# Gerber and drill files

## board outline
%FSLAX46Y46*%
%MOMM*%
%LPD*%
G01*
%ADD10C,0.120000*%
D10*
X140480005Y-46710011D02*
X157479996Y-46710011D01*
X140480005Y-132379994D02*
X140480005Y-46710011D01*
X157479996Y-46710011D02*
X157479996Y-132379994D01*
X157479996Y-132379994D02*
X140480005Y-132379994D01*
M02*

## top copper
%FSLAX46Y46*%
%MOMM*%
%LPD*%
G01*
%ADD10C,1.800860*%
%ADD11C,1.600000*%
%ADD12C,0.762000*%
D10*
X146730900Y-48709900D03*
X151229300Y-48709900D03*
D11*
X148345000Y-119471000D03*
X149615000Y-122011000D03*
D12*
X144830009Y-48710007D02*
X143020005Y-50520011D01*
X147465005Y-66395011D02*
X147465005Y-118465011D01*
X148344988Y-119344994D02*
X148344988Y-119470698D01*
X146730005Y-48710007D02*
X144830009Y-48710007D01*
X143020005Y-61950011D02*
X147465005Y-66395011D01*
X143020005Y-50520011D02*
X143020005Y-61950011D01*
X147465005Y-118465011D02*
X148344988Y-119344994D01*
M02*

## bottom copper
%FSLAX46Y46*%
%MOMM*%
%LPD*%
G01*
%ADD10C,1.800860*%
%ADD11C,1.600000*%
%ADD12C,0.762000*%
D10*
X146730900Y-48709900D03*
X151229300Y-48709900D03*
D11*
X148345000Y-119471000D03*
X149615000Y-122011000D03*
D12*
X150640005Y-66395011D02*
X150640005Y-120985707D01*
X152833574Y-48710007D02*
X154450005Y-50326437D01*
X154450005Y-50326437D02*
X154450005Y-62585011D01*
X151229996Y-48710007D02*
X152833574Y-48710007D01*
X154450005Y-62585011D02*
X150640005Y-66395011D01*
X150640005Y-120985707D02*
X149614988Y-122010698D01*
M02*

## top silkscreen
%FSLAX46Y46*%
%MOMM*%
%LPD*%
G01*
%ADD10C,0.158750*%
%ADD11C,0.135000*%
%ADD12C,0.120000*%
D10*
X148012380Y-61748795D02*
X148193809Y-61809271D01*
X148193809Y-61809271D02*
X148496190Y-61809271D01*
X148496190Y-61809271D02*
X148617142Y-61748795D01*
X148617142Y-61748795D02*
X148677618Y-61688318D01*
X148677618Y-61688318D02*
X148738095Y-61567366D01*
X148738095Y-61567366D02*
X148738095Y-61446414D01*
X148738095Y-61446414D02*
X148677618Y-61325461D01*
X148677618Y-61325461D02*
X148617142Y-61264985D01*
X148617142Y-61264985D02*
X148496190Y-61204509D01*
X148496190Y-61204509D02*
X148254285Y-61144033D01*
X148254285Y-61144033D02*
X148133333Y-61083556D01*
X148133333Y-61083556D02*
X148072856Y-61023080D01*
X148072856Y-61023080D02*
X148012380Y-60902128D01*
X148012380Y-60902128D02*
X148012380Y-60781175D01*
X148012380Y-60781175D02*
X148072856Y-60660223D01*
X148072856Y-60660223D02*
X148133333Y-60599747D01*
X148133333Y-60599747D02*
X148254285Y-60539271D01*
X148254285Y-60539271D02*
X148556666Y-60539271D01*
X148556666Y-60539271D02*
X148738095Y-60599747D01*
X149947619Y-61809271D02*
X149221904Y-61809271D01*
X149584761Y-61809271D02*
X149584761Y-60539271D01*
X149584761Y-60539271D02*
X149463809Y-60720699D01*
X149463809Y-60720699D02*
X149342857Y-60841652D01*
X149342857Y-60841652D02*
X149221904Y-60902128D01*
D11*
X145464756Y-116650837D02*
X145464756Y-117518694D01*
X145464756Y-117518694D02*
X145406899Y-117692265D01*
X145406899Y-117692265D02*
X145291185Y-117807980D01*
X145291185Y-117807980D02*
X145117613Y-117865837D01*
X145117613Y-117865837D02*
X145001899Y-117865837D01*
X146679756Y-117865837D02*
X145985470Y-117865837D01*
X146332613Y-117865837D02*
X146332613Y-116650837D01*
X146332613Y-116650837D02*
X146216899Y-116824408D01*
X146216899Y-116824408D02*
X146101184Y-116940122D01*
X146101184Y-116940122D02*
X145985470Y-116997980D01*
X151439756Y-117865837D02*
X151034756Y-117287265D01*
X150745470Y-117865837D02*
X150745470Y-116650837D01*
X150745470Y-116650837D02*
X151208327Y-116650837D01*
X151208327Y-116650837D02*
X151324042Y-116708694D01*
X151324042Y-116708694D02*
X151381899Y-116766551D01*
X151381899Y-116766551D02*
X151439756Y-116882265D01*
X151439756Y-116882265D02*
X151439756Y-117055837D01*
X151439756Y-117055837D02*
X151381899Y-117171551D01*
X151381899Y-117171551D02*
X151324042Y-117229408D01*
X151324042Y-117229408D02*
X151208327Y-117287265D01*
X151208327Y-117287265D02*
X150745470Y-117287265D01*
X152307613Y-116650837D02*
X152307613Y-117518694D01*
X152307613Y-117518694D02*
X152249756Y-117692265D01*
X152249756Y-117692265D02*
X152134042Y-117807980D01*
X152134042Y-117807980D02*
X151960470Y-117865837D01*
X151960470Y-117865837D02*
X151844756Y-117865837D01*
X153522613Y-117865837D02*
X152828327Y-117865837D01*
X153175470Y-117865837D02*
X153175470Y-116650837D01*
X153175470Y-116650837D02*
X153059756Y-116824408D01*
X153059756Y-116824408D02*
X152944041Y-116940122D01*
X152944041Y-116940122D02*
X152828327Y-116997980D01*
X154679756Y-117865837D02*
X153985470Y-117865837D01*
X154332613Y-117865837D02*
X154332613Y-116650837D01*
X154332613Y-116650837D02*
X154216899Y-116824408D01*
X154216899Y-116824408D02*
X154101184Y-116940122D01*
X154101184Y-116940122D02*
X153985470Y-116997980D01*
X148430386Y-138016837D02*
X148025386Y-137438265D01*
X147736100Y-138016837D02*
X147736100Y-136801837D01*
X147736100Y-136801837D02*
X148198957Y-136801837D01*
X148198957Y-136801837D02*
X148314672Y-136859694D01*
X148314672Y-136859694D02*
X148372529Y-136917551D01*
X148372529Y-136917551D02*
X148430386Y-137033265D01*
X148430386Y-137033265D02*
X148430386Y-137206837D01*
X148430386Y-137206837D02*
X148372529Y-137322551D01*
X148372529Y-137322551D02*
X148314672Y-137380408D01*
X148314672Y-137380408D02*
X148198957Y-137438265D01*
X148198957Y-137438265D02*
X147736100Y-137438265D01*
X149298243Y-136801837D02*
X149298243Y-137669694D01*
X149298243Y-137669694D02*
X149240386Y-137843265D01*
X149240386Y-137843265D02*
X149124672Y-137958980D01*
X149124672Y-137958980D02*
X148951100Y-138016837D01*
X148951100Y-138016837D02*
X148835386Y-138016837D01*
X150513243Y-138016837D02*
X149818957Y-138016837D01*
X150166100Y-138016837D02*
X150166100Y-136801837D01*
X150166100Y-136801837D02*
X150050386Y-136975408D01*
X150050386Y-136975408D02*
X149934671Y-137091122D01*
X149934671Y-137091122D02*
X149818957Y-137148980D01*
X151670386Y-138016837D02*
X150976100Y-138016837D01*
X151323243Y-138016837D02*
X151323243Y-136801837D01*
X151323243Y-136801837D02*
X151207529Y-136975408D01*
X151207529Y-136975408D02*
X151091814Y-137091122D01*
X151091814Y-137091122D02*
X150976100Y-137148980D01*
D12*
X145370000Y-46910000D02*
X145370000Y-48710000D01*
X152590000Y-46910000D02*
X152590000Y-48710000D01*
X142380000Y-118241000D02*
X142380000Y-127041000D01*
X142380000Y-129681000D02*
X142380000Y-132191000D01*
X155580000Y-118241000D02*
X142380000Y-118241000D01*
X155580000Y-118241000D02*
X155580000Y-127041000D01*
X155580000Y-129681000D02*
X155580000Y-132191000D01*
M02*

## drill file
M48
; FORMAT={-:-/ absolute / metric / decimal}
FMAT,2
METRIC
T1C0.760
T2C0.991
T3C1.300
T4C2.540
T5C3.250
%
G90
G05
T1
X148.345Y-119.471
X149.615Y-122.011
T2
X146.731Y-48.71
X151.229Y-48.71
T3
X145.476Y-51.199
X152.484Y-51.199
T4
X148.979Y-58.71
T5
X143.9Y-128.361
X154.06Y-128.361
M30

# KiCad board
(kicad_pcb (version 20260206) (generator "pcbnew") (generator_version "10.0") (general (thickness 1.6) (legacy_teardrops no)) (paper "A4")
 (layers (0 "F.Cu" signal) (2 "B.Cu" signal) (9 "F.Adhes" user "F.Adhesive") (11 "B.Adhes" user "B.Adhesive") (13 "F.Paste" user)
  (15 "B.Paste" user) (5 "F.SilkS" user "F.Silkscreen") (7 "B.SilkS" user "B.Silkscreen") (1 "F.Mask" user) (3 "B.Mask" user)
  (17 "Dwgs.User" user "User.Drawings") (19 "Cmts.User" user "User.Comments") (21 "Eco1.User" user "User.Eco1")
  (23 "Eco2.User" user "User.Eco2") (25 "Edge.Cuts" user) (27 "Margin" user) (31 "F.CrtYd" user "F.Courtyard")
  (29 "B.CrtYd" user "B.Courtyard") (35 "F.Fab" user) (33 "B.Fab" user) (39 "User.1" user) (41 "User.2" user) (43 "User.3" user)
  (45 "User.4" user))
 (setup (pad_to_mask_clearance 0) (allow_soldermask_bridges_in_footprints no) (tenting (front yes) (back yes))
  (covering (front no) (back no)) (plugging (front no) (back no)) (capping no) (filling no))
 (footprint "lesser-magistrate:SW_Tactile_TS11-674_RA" (layer "F.Cu") (at 148.98 48.71 180)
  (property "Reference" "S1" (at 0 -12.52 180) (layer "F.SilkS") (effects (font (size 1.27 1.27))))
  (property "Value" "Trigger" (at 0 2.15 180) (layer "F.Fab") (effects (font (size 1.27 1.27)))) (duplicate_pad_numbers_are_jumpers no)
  (fp_line (start 3.61 1.8) (end 3.61 0) (stroke (width 0.12) (type solid)) (layer "F.SilkS"))
  (fp_line (start -3.61 1.8) (end -3.61 0) (stroke (width 0.12) (type solid)) (layer "F.SilkS"))
  (pad "" np_thru_hole circle (at -3.504 -2.4891 180) (size 1.30048 1.30048) (drill 1.30048) (layers "*.Cu" "*.Mask"))
  (pad "" np_thru_hole circle (at 0.0012 -9.9999 180) (size 2.54 2.54) (drill 2.54) (layers "*.Cu" "*.Mask"))
  (pad "" np_thru_hole circle (at 3.5038 -2.4891 180) (size 1.30048 1.30048) (drill 1.30048) (layers "*.Cu" "*.Mask"))
  (pad "1" thru_hole circle (at 2.2491 0.0001 180) (size 1.80086 1.80086) (drill 0.990599) (layers "*.Cu" "*.Mask")
   (remove_unused_layers no) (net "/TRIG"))
  (pad "2" thru_hole circle (at -2.2493 0.0001 180) (size 1.80086 1.80086) (drill 0.990599) (layers "*.Cu" "*.Mask")
   (remove_unused_layers no) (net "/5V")))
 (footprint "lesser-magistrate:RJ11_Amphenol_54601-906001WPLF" (layer "F.Cu") (at 148.98 136.241)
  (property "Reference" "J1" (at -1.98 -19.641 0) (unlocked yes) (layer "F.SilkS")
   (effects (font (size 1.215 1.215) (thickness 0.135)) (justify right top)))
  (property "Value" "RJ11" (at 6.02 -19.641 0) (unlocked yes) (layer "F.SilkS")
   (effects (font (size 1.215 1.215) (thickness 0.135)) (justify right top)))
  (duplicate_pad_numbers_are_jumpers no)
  (fp_line (start -6.6 -18) (end -6.6 -9.2) (stroke (width 0.12) (type solid)) (layer "F.SilkS"))
  (fp_line (start -6.6 -6.56) (end -6.6 -4.05) (stroke (width 0.12) (type solid)) (layer "F.SilkS"))
  (fp_line (start 6.6 -18) (end -6.6 -18) (stroke (width 0.12) (type solid)) (layer "F.SilkS"))
  (fp_line (start 6.6 -18) (end 6.6 -9.2) (stroke (width 0.12) (type solid)) (layer "F.SilkS"))
  (fp_line (start 6.6 -6.56) (end 6.6 -4.05) (stroke (width 0.12) (type solid)) (layer "F.SilkS"))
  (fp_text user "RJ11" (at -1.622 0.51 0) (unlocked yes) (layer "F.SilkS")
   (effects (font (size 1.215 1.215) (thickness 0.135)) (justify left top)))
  (pad "" np_thru_hole circle (at -5.08 -7.88) (size 3.25 3.25) (drill 3.25) (layers "*.Cu" "*.Mask") (clearance 0.508))
  (pad "" np_thru_hole circle (at 5.08 -7.88) (size 3.25 3.25) (drill 3.25) (layers "*.Cu" "*.Mask") (clearance 0.508))
  (pad "3" thru_hole circle (at -0.635 -16.77) (size 1.6 1.6) (drill 0.76) (layers "*.Cu" "*.Mask") (remove_unused_layers no) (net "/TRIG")
   (solder_mask_margin 0.0508) (zone_connect 2) (thermal_bridge_angle 0))
  (pad "4" thru_hole circle (at 0.635 -14.23) (size 1.6 1.6) (drill 0.76) (layers "*.Cu" "*.Mask") (remove_unused_layers no) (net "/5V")
   (solder_mask_margin 0.0508) (zone_connect 2) (thermal_bridge_angle 0)))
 (gr_line (start 140.480005 46.710011) (end 157.479996 46.710011) (stroke (width 0.12) (type default)) (layer "Edge.Cuts"))
 (gr_line (start 140.480005 132.379994) (end 140.480005 46.710011) (stroke (width 0.12) (type default)) (layer "Edge.Cuts"))
 (gr_line (start 157.479996 46.710011) (end 157.479996 132.379994) (stroke (width 0.12) (type default)) (layer "Edge.Cuts"))
 (gr_line (start 157.479996 132.379994) (end 140.480005 132.379994) (stroke (width 0.12) (type default)) (layer "Edge.Cuts"))
 (segment (start 144.830009 48.710007) (end 143.020005 50.520011) (width 0.762) (layer "F.Cu") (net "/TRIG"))
 (segment (start 147.465005 66.395011) (end 147.465005 118.465011) (width 0.762) (layer "F.Cu") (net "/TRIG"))
 (segment (start 148.344988 119.344994) (end 148.344988 119.470698) (width 0.762) (layer "F.Cu") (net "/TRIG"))
 (segment (start 146.730005 48.710007) (end 144.830009 48.710007) (width 0.762) (layer "F.Cu") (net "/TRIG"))
 (segment (start 143.020005 61.950011) (end 147.465005 66.395011) (width 0.762) (layer "F.Cu") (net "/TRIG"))
 (segment (start 143.020005 50.520011) (end 143.020005 61.950011) (width 0.762) (layer "F.Cu") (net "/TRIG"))
 (segment (start 147.465005 118.465011) (end 148.344988 119.344994) (width 0.762) (layer "F.Cu") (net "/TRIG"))
 (segment (start 150.640005 66.395011) (end 150.640005 120.985707) (width 0.762) (layer "B.Cu") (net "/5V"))
 (segment (start 152.833574 48.710007) (end 154.450005 50.326437) (width 0.762) (layer "B.Cu") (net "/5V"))
 (segment (start 154.450005 50.326437) (end 154.450005 62.585011) (width 0.762) (layer "B.Cu") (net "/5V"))
 (segment (start 151.229996 48.710007) (end 152.833574 48.710007) (width 0.762) (layer "B.Cu") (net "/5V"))
 (segment (start 154.450005 62.585011) (end 150.640005 66.395011) (width 0.762) (layer "B.Cu") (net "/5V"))
 (segment (start 150.640005 120.985707) (end 149.614988 122.010698) (width 0.762) (layer "B.Cu") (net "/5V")))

